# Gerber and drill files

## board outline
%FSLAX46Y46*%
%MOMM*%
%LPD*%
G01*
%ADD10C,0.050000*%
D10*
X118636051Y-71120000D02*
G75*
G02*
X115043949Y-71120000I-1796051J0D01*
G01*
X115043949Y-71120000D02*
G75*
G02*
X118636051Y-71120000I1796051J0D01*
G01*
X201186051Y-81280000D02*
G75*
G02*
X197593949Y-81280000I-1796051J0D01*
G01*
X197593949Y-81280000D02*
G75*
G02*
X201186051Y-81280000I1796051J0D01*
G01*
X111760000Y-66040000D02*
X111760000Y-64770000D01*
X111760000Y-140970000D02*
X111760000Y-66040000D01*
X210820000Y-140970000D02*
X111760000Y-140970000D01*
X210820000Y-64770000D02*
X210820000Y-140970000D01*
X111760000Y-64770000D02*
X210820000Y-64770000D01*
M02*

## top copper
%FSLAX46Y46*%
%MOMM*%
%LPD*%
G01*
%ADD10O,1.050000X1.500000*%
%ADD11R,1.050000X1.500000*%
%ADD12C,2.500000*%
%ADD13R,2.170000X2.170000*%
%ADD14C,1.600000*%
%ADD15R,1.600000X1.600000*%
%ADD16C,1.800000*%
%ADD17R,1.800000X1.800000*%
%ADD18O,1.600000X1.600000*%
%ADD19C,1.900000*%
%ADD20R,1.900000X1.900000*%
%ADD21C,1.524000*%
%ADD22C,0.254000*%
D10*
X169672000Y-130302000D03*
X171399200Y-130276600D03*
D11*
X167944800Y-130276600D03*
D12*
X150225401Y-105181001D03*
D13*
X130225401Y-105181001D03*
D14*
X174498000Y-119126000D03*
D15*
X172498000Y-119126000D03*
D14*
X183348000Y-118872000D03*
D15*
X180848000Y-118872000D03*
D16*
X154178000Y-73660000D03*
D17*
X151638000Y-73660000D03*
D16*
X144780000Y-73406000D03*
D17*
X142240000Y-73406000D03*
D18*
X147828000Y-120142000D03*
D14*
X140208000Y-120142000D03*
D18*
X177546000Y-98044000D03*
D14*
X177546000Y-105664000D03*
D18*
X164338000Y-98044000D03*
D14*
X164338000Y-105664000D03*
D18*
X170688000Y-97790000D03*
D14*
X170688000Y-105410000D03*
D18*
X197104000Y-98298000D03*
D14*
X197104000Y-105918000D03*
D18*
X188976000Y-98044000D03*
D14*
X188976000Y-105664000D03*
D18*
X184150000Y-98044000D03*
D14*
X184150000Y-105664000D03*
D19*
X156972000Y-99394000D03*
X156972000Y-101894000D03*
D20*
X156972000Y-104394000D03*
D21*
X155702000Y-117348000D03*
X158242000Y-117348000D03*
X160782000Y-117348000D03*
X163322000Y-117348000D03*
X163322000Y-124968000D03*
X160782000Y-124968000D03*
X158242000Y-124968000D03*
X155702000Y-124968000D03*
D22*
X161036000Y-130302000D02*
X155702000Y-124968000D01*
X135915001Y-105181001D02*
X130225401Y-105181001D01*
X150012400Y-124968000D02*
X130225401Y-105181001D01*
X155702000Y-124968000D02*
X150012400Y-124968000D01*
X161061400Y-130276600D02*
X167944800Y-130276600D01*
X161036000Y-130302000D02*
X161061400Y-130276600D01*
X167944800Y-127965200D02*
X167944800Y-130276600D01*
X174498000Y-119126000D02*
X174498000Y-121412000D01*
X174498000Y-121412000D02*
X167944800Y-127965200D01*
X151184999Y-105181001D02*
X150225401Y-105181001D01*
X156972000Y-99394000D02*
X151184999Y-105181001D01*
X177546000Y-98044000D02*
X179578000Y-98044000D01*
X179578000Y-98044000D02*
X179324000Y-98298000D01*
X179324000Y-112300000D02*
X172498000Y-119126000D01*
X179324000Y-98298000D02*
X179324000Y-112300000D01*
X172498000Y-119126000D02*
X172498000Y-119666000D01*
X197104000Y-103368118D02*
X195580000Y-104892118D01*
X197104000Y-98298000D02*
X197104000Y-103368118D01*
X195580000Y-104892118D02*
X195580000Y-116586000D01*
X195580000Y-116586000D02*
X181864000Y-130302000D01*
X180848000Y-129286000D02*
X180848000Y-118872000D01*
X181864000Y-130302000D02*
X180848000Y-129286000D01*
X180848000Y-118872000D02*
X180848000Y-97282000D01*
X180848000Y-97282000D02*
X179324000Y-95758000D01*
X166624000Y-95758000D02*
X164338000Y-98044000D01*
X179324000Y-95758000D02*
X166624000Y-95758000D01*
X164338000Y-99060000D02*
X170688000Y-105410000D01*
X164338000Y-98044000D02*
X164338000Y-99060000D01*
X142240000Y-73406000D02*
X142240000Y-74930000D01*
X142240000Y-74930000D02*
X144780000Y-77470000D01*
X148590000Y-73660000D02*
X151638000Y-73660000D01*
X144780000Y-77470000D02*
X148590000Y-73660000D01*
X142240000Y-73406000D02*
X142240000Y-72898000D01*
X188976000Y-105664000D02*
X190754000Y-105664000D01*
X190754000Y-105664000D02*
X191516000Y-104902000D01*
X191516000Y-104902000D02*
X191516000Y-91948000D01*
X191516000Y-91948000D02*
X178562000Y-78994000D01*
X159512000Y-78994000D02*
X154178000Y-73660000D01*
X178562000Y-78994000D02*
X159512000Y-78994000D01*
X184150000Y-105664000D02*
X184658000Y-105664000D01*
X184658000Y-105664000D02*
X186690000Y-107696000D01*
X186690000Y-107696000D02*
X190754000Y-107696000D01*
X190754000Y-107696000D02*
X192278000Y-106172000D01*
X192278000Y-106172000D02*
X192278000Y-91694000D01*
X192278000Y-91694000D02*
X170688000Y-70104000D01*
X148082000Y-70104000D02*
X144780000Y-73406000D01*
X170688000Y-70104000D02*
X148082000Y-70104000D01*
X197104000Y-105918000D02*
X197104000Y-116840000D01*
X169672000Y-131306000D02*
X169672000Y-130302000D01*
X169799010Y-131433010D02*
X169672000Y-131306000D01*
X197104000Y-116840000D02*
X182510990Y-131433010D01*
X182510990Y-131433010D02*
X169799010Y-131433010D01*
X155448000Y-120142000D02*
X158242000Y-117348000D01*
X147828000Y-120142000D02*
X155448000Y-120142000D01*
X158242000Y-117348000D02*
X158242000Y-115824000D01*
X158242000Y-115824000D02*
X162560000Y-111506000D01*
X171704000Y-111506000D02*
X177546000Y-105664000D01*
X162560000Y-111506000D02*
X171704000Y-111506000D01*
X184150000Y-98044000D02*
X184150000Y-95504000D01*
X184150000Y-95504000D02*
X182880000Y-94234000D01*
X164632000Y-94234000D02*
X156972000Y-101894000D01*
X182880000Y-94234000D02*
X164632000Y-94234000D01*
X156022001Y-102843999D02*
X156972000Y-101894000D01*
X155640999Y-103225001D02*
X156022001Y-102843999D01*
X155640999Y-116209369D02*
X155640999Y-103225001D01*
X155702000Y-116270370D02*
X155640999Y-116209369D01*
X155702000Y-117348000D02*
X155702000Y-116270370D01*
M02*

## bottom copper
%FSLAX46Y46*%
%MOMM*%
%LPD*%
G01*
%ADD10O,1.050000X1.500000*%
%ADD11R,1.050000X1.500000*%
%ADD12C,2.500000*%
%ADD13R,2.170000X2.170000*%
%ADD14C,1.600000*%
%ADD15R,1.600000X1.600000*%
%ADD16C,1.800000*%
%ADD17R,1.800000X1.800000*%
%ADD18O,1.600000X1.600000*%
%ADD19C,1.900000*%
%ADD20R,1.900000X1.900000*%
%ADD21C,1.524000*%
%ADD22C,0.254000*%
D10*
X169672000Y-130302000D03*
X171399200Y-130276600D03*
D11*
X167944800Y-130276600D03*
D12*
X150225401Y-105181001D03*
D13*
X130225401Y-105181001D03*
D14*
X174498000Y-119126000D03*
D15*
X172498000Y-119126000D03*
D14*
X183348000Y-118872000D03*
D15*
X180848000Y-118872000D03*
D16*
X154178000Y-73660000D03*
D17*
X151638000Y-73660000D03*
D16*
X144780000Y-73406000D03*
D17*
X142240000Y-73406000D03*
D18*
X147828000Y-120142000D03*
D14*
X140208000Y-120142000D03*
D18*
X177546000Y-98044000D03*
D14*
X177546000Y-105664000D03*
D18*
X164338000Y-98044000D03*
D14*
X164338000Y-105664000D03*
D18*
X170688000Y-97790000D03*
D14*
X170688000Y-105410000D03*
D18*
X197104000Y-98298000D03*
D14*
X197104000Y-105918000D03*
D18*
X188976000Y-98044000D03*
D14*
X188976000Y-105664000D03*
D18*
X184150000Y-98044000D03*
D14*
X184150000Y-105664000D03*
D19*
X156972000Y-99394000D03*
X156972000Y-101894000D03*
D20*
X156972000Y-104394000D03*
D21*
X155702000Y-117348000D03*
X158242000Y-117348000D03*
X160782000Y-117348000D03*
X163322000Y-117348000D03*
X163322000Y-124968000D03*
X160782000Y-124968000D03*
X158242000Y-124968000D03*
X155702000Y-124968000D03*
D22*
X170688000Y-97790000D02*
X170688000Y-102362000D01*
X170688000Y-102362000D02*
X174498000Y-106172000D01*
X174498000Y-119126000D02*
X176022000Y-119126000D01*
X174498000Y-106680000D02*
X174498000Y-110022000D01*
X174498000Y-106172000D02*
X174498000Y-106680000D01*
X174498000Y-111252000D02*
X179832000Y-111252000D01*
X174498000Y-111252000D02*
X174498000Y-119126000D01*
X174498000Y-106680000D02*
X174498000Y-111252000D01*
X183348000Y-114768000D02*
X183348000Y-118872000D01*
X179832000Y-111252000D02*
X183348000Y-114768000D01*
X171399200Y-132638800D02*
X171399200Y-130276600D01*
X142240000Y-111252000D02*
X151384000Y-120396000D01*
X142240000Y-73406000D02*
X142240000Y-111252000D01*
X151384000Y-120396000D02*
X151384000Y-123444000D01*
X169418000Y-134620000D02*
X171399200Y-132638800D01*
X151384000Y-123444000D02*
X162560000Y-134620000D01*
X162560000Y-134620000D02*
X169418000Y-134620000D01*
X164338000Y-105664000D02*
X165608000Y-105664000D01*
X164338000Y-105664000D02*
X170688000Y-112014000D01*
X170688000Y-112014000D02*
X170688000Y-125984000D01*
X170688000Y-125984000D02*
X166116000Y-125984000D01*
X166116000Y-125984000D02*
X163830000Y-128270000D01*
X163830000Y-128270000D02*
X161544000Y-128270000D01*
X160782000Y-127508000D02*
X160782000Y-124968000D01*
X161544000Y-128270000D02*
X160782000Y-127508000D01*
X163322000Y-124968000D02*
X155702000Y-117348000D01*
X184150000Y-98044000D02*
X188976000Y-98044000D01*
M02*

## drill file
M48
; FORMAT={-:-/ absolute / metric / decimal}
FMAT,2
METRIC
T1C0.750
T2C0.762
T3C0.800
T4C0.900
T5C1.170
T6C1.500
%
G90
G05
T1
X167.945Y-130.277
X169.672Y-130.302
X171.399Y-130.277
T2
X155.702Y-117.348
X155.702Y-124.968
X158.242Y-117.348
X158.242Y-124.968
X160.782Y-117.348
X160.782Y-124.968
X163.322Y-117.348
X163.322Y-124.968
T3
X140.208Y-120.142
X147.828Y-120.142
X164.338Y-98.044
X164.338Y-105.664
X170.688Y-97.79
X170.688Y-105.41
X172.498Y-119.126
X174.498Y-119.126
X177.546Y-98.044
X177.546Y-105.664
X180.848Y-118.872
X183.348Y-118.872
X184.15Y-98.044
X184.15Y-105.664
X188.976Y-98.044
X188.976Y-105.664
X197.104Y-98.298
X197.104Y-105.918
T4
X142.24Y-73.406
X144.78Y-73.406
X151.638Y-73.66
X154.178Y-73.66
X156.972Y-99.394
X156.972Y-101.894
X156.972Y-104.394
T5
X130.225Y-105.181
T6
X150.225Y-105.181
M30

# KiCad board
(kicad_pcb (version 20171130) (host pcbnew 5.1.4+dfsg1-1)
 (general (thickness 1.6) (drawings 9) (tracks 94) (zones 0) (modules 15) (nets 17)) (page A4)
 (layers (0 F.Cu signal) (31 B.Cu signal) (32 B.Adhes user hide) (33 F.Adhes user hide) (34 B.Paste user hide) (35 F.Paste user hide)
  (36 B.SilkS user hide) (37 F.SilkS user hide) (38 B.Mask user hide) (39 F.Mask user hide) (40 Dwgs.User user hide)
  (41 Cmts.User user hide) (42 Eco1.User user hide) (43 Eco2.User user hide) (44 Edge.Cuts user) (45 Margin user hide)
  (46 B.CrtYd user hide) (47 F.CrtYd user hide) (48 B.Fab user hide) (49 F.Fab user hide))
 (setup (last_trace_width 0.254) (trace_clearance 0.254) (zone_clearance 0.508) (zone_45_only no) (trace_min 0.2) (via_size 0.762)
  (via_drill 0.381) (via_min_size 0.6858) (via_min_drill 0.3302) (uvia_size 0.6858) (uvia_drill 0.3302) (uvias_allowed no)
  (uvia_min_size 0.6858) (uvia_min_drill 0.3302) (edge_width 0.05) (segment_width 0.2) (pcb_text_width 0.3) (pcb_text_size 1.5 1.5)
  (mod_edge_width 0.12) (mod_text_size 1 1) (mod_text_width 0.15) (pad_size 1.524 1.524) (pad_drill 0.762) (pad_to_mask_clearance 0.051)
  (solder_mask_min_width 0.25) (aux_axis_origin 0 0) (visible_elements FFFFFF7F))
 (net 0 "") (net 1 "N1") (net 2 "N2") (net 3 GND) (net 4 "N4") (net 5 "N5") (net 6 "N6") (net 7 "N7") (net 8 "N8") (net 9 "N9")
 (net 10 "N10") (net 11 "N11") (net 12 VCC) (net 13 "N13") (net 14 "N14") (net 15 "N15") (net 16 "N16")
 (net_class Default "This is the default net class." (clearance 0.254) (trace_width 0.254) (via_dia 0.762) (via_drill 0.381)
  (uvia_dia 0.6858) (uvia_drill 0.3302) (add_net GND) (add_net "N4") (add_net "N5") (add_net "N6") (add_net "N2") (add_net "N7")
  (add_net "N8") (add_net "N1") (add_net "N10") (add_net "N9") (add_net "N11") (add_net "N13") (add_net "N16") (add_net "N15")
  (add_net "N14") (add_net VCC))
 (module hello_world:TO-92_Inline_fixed (layer F.Cu) (at 168.402 130.302)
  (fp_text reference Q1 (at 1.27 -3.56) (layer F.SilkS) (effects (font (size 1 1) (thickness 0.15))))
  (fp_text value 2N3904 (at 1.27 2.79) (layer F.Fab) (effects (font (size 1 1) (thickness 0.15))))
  (pad 2 thru_hole oval (at 1.27 0) (size 1.05 1.5) (drill 0.75) (layers *.Cu *.Mask) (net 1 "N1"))
  (pad 3 thru_hole oval (at 2.9972 -0.0254) (size 1.05 1.5) (drill 0.75) (layers *.Cu *.Mask) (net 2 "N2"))
  (pad 1 thru_hole rect (at -0.4572 -0.0254) (size 1.05 1.5) (drill 0.75) (layers *.Cu *.Mask) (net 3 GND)))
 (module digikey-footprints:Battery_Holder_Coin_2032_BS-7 (layer F.Cu) (at 130.225401 105.181001)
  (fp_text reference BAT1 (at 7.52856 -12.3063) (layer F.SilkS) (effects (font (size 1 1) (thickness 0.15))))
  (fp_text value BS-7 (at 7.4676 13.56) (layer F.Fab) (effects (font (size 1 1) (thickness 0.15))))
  (pad Pos thru_hole circle (at 20 0) (size 2.5 2.5) (drill 1.5) (layers *.Cu *.Mask) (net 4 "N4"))
  (pad Neg thru_hole rect (at 0 0) (size 2.17 2.17) (drill 1.17) (layers *.Cu *.Mask) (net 3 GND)))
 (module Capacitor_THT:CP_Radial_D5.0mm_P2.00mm (layer F.Cu) (at 172.498 119.126)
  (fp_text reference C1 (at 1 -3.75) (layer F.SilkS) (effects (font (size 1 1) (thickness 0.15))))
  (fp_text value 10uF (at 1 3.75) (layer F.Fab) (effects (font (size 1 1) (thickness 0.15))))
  (pad 2 thru_hole circle (at 2 0) (size 1.6 1.6) (drill 0.8) (layers *.Cu *.Mask) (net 3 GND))
  (pad 1 thru_hole rect (at 0 0) (size 1.6 1.6) (drill 0.8) (layers *.Cu *.Mask) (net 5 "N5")))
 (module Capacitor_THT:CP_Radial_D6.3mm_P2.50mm (layer F.Cu) (at 180.848 118.872)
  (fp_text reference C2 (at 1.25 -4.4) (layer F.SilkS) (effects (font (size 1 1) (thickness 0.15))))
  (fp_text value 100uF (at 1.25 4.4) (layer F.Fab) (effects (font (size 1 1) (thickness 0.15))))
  (pad 2 thru_hole circle (at 2.5 0) (size 1.6 1.6) (drill 0.8) (layers *.Cu *.Mask) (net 3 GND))
  (pad 1 thru_hole rect (at 0 0) (size 1.6 1.6) (drill 0.8) (layers *.Cu *.Mask) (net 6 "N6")))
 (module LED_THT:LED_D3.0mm (layer F.Cu) (at 151.638 73.66)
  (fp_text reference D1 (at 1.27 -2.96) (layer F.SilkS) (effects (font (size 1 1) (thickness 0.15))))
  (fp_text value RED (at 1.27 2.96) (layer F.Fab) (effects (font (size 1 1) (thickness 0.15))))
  (pad 2 thru_hole circle (at 2.54 0) (size 1.8 1.8) (drill 0.9) (layers *.Cu *.Mask) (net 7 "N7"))
  (pad 1 thru_hole rect (at 0 0) (size 1.8 1.8) (drill 0.9) (layers *.Cu *.Mask) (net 2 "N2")))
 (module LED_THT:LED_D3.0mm (layer F.Cu) (at 142.24 73.406)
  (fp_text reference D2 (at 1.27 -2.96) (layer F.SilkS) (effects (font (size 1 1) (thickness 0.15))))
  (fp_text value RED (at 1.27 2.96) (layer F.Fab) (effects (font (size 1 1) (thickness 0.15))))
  (pad 2 thru_hole circle (at 2.54 0) (size 1.8 1.8) (drill 0.9) (layers *.Cu *.Mask) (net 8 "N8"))
  (pad 1 thru_hole rect (at 0 0) (size 1.8 1.8) (drill 0.9) (layers *.Cu *.Mask) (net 2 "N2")))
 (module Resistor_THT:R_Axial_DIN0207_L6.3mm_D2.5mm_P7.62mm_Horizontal (layer F.Cu) (at 140.208 120.142)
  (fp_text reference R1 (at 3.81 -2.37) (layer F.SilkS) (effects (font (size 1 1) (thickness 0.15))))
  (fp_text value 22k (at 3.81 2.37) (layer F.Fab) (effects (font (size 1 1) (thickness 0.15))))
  (pad 2 thru_hole oval (at 7.62 0) (size 1.6 1.6) (drill 0.8) (layers *.Cu *.Mask) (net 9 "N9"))
  (pad 1 thru_hole circle (at 0 0) (size 1.6 1.6) (drill 0.8) (layers *.Cu *.Mask) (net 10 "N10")))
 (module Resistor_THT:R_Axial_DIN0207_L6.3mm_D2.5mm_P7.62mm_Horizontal (layer F.Cu) (at 177.546 105.664 90)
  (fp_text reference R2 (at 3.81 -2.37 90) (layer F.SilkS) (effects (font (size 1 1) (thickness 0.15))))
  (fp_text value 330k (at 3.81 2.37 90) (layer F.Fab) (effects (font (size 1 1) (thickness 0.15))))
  (pad 2 thru_hole oval (at 7.62 0 90) (size 1.6 1.6) (drill 0.8) (layers *.Cu *.Mask) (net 5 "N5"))
  (pad 1 thru_hole circle (at 0 0 90) (size 1.6 1.6) (drill 0.8) (layers *.Cu *.Mask) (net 9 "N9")))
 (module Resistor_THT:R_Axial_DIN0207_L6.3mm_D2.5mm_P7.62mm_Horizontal (layer F.Cu) (at 164.338 105.664 90)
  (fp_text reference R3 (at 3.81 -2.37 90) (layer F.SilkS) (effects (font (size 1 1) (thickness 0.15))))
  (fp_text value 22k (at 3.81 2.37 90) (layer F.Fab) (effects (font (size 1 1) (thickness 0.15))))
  (pad 2 thru_hole oval (at 7.62 0 90) (size 1.6 1.6) (drill 0.8) (layers *.Cu *.Mask) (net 6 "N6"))
  (pad 1 thru_hole circle (at 0 0 90) (size 1.6 1.6) (drill 0.8) (layers *.Cu *.Mask) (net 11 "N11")))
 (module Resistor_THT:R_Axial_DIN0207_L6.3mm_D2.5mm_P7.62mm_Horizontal (layer F.Cu) (at 170.688 105.41 90)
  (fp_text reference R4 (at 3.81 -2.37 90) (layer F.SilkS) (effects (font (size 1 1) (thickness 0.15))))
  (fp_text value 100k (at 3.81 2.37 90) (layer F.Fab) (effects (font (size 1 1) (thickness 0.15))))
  (pad 2 thru_hole oval (at 7.62 0 90) (size 1.6 1.6) (drill 0.8) (layers *.Cu *.Mask) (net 3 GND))
  (pad 1 thru_hole circle (at 0 0 90) (size 1.6 1.6) (drill 0.8) (layers *.Cu *.Mask) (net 6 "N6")))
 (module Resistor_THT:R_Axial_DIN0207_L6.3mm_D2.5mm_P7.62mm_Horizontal (layer F.Cu) (at 197.104 105.918 90)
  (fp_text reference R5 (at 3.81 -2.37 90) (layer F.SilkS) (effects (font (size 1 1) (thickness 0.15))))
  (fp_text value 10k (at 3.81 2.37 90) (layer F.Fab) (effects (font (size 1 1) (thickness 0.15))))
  (pad 2 thru_hole oval (at 7.62 0 90) (size 1.6 1.6) (drill 0.8) (layers *.Cu *.Mask) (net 6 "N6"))
  (pad 1 thru_hole circle (at 0 0 90) (size 1.6 1.6) (drill 0.8) (layers *.Cu *.Mask) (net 1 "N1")))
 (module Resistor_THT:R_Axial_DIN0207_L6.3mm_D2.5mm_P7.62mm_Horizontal (layer F.Cu) (at 188.976 105.664 90)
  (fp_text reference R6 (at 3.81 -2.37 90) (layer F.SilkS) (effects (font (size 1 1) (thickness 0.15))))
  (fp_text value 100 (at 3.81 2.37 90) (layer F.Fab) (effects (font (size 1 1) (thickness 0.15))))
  (pad 2 thru_hole oval (at 7.62 0 90) (size 1.6 1.6) (drill 0.8) (layers *.Cu *.Mask) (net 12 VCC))
  (pad 1 thru_hole circle (at 0 0 90) (size 1.6 1.6) (drill 0.8) (layers *.Cu *.Mask) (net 7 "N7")))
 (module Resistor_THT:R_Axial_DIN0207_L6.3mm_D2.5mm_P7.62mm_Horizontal (layer F.Cu) (at 184.15 105.664 90)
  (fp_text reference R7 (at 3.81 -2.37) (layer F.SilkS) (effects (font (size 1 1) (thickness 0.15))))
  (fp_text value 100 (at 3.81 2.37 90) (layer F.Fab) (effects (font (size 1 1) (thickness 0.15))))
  (pad 2 thru_hole oval (at 7.62 0 90) (size 1.6 1.6) (drill 0.8) (layers *.Cu *.Mask) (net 12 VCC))
  (pad 1 thru_hole circle (at 0 0 90) (size 1.6 1.6) (drill 0.8) (layers *.Cu *.Mask) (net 8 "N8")))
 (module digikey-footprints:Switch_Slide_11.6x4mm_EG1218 (layer F.Cu) (at 156.972 104.394 90)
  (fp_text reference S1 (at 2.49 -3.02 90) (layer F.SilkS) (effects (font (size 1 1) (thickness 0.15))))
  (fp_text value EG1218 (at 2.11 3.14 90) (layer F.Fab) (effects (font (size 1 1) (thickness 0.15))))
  (pad 3 thru_hole circle (at 5 0 90) (size 1.9 1.9) (drill 0.9) (layers *.Cu *.Mask) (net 4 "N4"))
  (pad 2 thru_hole circle (at 2.5 0 90) (size 1.9 1.9) (drill 0.9) (layers *.Cu *.Mask) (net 12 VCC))
  (pad 1 thru_hole rect (at 0 0 90) (size 1.9 1.9) (drill 0.9) (layers *.Cu *.Mask) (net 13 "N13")))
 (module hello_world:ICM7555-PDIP (layer F.Cu) (at 159.512 121.158)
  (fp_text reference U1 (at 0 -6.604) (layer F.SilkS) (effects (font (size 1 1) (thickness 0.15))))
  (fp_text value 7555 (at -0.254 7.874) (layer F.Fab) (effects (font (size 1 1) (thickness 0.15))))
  (pad 8 thru_hole circle (at -3.81 -3.81) (size 1.524 1.524) (drill 0.762) (layers *.Cu *.Mask) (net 12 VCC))
  (pad 7 thru_hole circle (at -1.27 -3.81) (size 1.524 1.524) (drill 0.762) (layers *.Cu *.Mask) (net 9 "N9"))
  (pad 6 thru_hole circle (at 1.27 -3.81) (size 1.524 1.524) (drill 0.762) (layers *.Cu *.Mask) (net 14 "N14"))
  (pad 5 thru_hole circle (at 3.81 -3.81) (size 1.524 1.524) (drill 0.762) (layers *.Cu *.Mask) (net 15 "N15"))
  (pad 4 thru_hole circle (at 3.81 3.81) (size 1.524 1.524) (drill 0.762) (layers *.Cu *.Mask) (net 12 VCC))
  (pad 3 thru_hole circle (at 1.27 3.81) (size 1.524 1.524) (drill 0.762) (layers *.Cu *.Mask) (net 11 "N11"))
  (pad 2 thru_hole circle (at -1.27 3.81) (size 1.524 1.524) (drill 0.762) (layers *.Cu *.Mask) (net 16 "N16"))
  (pad 1 thru_hole circle (at -3.81 3.81) (size 1.524 1.524) (drill 0.762) (layers *.Cu *.Mask) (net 3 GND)))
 (gr_circle (center 116.84 71.12) (end 118.11 72.39) (layer Edge.Cuts) (width 0.05))
 (gr_circle (center 199.39 81.28) (end 200.66 82.55) (layer Edge.Cuts) (width 0.05))
 (gr_line (start 111.76 66.04) (end 111.76 64.77) (layer Edge.Cuts) (width 0.05))
 (gr_line (start 111.76 140.97) (end 111.76 66.04) (layer Edge.Cuts) (width 0.05))
 (gr_line (start 210.82 140.97) (end 111.76 140.97) (layer Edge.Cuts) (width 0.05))
 (gr_line (start 210.82 64.77) (end 210.82 140.97) (layer Edge.Cuts) (width 0.05))
 (gr_line (start 111.76 64.77) (end 210.82 64.77) (layer Edge.Cuts) (width 0.05))
 (segment (start 161.036 130.302) (end 155.702 124.968) (width 0.254) (layer F.Cu) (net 3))
 (segment (start 135.915001 105.181001) (end 130.225401 105.181001) (width 0.254) (layer F.Cu) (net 3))
 (segment (start 150.0124 124.968) (end 130.225401 105.181001) (width 0.254) (layer F.Cu) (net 3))
 (segment (start 155.702 124.968) (end 150.0124 124.968) (width 0.254) (layer F.Cu) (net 3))
 (segment (start 170.688 97.79) (end 170.688 102.362) (width 0.254) (layer B.Cu) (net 3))
 (segment (start 170.688 102.362) (end 174.498 106.172) (width 0.254) (layer B.Cu) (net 3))
 (segment (start 174.498 119.126) (end 176.022 119.126) (width 0.254) (layer B.Cu) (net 3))
 (segment (start 174.498 106.68) (end 174.498 110.022) (width 0.254) (layer B.Cu) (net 3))
 (segment (start 174.498 106.172) (end 174.498 106.68) (width 0.254) (layer B.Cu) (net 3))
 (segment (start 161.0614 130.2766) (end 167.9448 130.2766) (width 0.254) (layer F.Cu) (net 3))
 (segment (start 161.036 130.302) (end 161.0614 130.2766) (width 0.254) (layer F.Cu) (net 3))
 (segment (start 167.9448 127.9652) (end 167.9448 130.2766) (width 0.254) (layer F.Cu) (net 3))
 (segment (start 174.498 119.126) (end 174.498 121.412) (width 0.254) (layer F.Cu) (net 3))
 (segment (start 174.498 121.412) (end 167.9448 127.9652) (width 0.254) (layer F.Cu) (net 3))
 (segment (start 174.498 111.252) (end 179.832 111.252) (width 0.254) (layer B.Cu) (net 3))
 (segment (start 174.498 111.252) (end 174.498 119.126) (width 0.254) (layer B.Cu) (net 3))
 (segment (start 174.498 106.68) (end 174.498 111.252) (width 0.254) (layer B.Cu) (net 3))
 (segment (start 183.348 114.768) (end 183.348 118.872) (width 0.254) (layer B.Cu) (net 3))
 (segment (start 179.832 111.252) (end 183.348 114.768) (width 0.254) (layer B.Cu) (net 3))
 (segment (start 151.184999 105.181001) (end 150.225401 105.181001) (width 0.254) (layer F.Cu) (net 4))
 (segment (start 156.972 99.394) (end 151.184999 105.181001) (width 0.254) (layer F.Cu) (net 4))
 (segment (start 177.546 98.044) (end 179.578 98.044) (width 0.254) (layer F.Cu) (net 5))
 (segment (start 179.578 98.044) (end 179.324 98.298) (width 0.254) (layer F.Cu) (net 5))
 (segment (start 179.324 112.3) (end 172.498 119.126) (width 0.254) (layer F.Cu) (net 5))
 (segment (start 179.324 98.298) (end 179.324 112.3) (width 0.254) (layer F.Cu) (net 5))
 (segment (start 172.498 119.126) (end 172.498 119.666) (width 0.254) (layer F.Cu) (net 5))
 (segment (start 197.104 103.368118) (end 195.58 104.892118) (width 0.254) (layer F.Cu) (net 6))
 (segment (start 197.104 98.298) (end 197.104 103.368118) (width 0.254) (layer F.Cu) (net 6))
 (segment (start 195.58 104.892118) (end 195.58 116.586) (width 0.254) (layer F.Cu) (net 6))
 (segment (start 195.58 116.586) (end 181.864 130.302) (width 0.254) (layer F.Cu) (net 6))
 (segment (start 180.848 129.286) (end 180.848 118.872) (width 0.254) (layer F.Cu) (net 6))
 (segment (start 181.864 130.302) (end 180.848 129.286) (width 0.254) (layer F.Cu) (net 6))
 (segment (start 180.848 118.872) (end 180.848 97.282) (width 0.254) (layer F.Cu) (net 6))
 (segment (start 180.848 97.282) (end 179.324 95.758) (width 0.254) (layer F.Cu) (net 6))
 (segment (start 166.624 95.758) (end 164.338 98.044) (width 0.254) (layer F.Cu) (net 6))
 (segment (start 179.324 95.758) (end 166.624 95.758) (width 0.254) (layer F.Cu) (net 6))
 (segment (start 164.338 99.06) (end 170.688 105.41) (width 0.254) (layer F.Cu) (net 6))
 (segment (start 164.338 98.044) (end 164.338 99.06) (width 0.254) (layer F.Cu) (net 6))
 (segment (start 142.24 73.406) (end 142.24 74.93) (width 0.254) (layer F.Cu) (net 2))
 (segment (start 142.24 74.93) (end 144.78 77.47) (width 0.254) (layer F.Cu) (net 2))
 (segment (start 148.59 73.66) (end 151.638 73.66) (width 0.254) (layer F.Cu) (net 2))
 (segment (start 144.78 77.47) (end 148.59 73.66) (width 0.254) (layer F.Cu) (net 2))
 (segment (start 142.24 73.406) (end 142.24 72.898) (width 0.254) (layer F.Cu) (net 2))
 (segment (start 171.3992 132.6388) (end 171.3992 130.2766) (width 0.254) (layer B.Cu) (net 2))
 (segment (start 142.24 111.252) (end 151.384 120.396) (width 0.254) (layer B.Cu) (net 2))
 (segment (start 142.24 73.406) (end 142.24 111.252) (width 0.254) (layer B.Cu) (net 2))
 (segment (start 151.384 120.396) (end 151.384 123.444) (width 0.254) (layer B.Cu) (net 2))
 (segment (start 169.418 134.62) (end 171.3992 132.6388) (width 0.254) (layer B.Cu) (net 2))
 (segment (start 151.384 123.444) (end 162.56 134.62) (width 0.254) (layer B.Cu) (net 2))
 (segment (start 162.56 134.62) (end 169.418 134.62) (width 0.254) (layer B.Cu) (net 2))
 (segment (start 188.976 105.664) (end 190.754 105.664) (width 0.254) (layer F.Cu) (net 7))
 (segment (start 190.754 105.664) (end 191.516 104.902) (width 0.254) (layer F.Cu) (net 7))
 (segment (start 191.516 104.902) (end 191.516 91.948) (width 0.254) (layer F.Cu) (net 7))
 (segment (start 191.516 91.948) (end 178.562 78.994) (width 0.254) (layer F.Cu) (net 7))
 (segment (start 159.512 78.994) (end 154.178 73.66) (width 0.254) (layer F.Cu) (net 7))
 (segment (start 178.562 78.994) (end 159.512 78.994) (width 0.254) (layer F.Cu) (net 7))
 (segment (start 184.15 105.664) (end 184.658 105.664) (width 0.254) (layer F.Cu) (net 8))
 (segment (start 184.658 105.664) (end 186.69 107.696) (width 0.254) (layer F.Cu) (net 8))
 (segment (start 186.69 107.696) (end 190.754 107.696) (width 0.254) (layer F.Cu) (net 8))
 (segment (start 190.754 107.696) (end 192.278 106.172) (width 0.254) (layer F.Cu) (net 8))
 (segment (start 192.278 106.172) (end 192.278 91.694) (width 0.254) (layer F.Cu) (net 8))
 (segment (start 192.278 91.694) (end 170.688 70.104) (width 0.254) (layer F.Cu) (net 8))
 (segment (start 148.082 70.104) (end 144.78 73.406) (width 0.254) (layer F.Cu) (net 8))
 (segment (start 170.688 70.104) (end 148.082 70.104) (width 0.254) (layer F.Cu) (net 8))
 (segment (start 197.104 105.918) (end 197.104 116.84) (width 0.254) (layer F.Cu) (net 1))
 (segment (start 169.672 131.306) (end 169.672 130.302) (width 0.254) (layer F.Cu) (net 1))
 (segment (start 169.79901 131.43301) (end 169.672 131.306) (width 0.254) (layer F.Cu) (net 1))
 (segment (start 197.104 116.84) (end 182.51099 131.43301) (width 0.254) (layer F.Cu) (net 1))
 (segment (start 182.51099 131.43301) (end 169.79901 131.43301) (width 0.254) (layer F.Cu) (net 1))
 (segment (start 155.448 120.142) (end 158.242 117.348) (width 0.254) (layer F.Cu) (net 9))
 (segment (start 147.828 120.142) (end 155.448 120.142) (width 0.254) (layer F.Cu) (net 9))
 (segment (start 158.242 117.348) (end 158.242 115.824) (width 0.254) (layer F.Cu) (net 9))
 (segment (start 158.242 115.824) (end 162.56 111.506) (width 0.254) (layer F.Cu) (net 9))
 (segment (start 171.704 111.506) (end 177.546 105.664) (width 0.254) (layer F.Cu) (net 9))
 (segment (start 162.56 111.506) (end 171.704 111.506) (width 0.254) (layer F.Cu) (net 9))
 (segment (start 164.338 105.664) (end 165.608 105.664) (width 0.254) (layer B.Cu) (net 11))
 (segment (start 164.338 105.664) (end 170.688 112.014) (width 0.254) (layer B.Cu) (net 11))
 (segment (start 170.688 112.014) (end 170.688 125.984) (width 0.254) (layer B.Cu) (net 11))
 (segment (start 170.688 125.984) (end 166.116 125.984) (width 0.254) (layer B.Cu) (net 11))
 (segment (start 166.116 125.984) (end 163.83 128.27) (width 0.254) (layer B.Cu) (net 11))
 (segment (start 163.83 128.27) (end 161.544 128.27) (width 0.254) (layer B.Cu) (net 11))
 (segment (start 160.782 127.508) (end 160.782 124.968) (width 0.254) (layer B.Cu) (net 11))
 (segment (start 161.544 128.27) (end 160.782 127.508) (width 0.254) (layer B.Cu) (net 11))
 (segment (start 184.15 98.044) (end 184.15 95.504) (width 0.254) (layer F.Cu) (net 12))
 (segment (start 184.15 95.504) (end 182.88 94.234) (width 0.254) (layer F.Cu) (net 12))
 (segment (start 164.632 94.234) (end 156.972 101.894) (width 0.254) (layer F.Cu) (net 12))
 (segment (start 182.88 94.234) (end 164.632 94.234) (width 0.254) (layer F.Cu) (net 12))
 (segment (start 156.022001 102.843999) (end 156.972 101.894) (width 0.254) (layer F.Cu) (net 12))
 (segment (start 155.640999 103.225001) (end 156.022001 102.843999) (width 0.254) (layer F.Cu) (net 12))
 (segment (start 155.640999 116.209369) (end 155.640999 103.225001) (width 0.254) (layer F.Cu) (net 12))
 (segment (start 155.702 116.27037) (end 155.640999 116.209369) (width 0.254) (layer F.Cu) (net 12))
 (segment (start 155.702 117.348) (end 155.702 116.27037) (width 0.254) (layer F.Cu) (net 12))
 (segment (start 163.322 124.968) (end 155.702 117.348) (width 0.254) (layer B.Cu) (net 12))
 (segment (start 184.15 98.044) (end 188.976 98.044) (width 0.254) (layer B.Cu) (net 12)))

